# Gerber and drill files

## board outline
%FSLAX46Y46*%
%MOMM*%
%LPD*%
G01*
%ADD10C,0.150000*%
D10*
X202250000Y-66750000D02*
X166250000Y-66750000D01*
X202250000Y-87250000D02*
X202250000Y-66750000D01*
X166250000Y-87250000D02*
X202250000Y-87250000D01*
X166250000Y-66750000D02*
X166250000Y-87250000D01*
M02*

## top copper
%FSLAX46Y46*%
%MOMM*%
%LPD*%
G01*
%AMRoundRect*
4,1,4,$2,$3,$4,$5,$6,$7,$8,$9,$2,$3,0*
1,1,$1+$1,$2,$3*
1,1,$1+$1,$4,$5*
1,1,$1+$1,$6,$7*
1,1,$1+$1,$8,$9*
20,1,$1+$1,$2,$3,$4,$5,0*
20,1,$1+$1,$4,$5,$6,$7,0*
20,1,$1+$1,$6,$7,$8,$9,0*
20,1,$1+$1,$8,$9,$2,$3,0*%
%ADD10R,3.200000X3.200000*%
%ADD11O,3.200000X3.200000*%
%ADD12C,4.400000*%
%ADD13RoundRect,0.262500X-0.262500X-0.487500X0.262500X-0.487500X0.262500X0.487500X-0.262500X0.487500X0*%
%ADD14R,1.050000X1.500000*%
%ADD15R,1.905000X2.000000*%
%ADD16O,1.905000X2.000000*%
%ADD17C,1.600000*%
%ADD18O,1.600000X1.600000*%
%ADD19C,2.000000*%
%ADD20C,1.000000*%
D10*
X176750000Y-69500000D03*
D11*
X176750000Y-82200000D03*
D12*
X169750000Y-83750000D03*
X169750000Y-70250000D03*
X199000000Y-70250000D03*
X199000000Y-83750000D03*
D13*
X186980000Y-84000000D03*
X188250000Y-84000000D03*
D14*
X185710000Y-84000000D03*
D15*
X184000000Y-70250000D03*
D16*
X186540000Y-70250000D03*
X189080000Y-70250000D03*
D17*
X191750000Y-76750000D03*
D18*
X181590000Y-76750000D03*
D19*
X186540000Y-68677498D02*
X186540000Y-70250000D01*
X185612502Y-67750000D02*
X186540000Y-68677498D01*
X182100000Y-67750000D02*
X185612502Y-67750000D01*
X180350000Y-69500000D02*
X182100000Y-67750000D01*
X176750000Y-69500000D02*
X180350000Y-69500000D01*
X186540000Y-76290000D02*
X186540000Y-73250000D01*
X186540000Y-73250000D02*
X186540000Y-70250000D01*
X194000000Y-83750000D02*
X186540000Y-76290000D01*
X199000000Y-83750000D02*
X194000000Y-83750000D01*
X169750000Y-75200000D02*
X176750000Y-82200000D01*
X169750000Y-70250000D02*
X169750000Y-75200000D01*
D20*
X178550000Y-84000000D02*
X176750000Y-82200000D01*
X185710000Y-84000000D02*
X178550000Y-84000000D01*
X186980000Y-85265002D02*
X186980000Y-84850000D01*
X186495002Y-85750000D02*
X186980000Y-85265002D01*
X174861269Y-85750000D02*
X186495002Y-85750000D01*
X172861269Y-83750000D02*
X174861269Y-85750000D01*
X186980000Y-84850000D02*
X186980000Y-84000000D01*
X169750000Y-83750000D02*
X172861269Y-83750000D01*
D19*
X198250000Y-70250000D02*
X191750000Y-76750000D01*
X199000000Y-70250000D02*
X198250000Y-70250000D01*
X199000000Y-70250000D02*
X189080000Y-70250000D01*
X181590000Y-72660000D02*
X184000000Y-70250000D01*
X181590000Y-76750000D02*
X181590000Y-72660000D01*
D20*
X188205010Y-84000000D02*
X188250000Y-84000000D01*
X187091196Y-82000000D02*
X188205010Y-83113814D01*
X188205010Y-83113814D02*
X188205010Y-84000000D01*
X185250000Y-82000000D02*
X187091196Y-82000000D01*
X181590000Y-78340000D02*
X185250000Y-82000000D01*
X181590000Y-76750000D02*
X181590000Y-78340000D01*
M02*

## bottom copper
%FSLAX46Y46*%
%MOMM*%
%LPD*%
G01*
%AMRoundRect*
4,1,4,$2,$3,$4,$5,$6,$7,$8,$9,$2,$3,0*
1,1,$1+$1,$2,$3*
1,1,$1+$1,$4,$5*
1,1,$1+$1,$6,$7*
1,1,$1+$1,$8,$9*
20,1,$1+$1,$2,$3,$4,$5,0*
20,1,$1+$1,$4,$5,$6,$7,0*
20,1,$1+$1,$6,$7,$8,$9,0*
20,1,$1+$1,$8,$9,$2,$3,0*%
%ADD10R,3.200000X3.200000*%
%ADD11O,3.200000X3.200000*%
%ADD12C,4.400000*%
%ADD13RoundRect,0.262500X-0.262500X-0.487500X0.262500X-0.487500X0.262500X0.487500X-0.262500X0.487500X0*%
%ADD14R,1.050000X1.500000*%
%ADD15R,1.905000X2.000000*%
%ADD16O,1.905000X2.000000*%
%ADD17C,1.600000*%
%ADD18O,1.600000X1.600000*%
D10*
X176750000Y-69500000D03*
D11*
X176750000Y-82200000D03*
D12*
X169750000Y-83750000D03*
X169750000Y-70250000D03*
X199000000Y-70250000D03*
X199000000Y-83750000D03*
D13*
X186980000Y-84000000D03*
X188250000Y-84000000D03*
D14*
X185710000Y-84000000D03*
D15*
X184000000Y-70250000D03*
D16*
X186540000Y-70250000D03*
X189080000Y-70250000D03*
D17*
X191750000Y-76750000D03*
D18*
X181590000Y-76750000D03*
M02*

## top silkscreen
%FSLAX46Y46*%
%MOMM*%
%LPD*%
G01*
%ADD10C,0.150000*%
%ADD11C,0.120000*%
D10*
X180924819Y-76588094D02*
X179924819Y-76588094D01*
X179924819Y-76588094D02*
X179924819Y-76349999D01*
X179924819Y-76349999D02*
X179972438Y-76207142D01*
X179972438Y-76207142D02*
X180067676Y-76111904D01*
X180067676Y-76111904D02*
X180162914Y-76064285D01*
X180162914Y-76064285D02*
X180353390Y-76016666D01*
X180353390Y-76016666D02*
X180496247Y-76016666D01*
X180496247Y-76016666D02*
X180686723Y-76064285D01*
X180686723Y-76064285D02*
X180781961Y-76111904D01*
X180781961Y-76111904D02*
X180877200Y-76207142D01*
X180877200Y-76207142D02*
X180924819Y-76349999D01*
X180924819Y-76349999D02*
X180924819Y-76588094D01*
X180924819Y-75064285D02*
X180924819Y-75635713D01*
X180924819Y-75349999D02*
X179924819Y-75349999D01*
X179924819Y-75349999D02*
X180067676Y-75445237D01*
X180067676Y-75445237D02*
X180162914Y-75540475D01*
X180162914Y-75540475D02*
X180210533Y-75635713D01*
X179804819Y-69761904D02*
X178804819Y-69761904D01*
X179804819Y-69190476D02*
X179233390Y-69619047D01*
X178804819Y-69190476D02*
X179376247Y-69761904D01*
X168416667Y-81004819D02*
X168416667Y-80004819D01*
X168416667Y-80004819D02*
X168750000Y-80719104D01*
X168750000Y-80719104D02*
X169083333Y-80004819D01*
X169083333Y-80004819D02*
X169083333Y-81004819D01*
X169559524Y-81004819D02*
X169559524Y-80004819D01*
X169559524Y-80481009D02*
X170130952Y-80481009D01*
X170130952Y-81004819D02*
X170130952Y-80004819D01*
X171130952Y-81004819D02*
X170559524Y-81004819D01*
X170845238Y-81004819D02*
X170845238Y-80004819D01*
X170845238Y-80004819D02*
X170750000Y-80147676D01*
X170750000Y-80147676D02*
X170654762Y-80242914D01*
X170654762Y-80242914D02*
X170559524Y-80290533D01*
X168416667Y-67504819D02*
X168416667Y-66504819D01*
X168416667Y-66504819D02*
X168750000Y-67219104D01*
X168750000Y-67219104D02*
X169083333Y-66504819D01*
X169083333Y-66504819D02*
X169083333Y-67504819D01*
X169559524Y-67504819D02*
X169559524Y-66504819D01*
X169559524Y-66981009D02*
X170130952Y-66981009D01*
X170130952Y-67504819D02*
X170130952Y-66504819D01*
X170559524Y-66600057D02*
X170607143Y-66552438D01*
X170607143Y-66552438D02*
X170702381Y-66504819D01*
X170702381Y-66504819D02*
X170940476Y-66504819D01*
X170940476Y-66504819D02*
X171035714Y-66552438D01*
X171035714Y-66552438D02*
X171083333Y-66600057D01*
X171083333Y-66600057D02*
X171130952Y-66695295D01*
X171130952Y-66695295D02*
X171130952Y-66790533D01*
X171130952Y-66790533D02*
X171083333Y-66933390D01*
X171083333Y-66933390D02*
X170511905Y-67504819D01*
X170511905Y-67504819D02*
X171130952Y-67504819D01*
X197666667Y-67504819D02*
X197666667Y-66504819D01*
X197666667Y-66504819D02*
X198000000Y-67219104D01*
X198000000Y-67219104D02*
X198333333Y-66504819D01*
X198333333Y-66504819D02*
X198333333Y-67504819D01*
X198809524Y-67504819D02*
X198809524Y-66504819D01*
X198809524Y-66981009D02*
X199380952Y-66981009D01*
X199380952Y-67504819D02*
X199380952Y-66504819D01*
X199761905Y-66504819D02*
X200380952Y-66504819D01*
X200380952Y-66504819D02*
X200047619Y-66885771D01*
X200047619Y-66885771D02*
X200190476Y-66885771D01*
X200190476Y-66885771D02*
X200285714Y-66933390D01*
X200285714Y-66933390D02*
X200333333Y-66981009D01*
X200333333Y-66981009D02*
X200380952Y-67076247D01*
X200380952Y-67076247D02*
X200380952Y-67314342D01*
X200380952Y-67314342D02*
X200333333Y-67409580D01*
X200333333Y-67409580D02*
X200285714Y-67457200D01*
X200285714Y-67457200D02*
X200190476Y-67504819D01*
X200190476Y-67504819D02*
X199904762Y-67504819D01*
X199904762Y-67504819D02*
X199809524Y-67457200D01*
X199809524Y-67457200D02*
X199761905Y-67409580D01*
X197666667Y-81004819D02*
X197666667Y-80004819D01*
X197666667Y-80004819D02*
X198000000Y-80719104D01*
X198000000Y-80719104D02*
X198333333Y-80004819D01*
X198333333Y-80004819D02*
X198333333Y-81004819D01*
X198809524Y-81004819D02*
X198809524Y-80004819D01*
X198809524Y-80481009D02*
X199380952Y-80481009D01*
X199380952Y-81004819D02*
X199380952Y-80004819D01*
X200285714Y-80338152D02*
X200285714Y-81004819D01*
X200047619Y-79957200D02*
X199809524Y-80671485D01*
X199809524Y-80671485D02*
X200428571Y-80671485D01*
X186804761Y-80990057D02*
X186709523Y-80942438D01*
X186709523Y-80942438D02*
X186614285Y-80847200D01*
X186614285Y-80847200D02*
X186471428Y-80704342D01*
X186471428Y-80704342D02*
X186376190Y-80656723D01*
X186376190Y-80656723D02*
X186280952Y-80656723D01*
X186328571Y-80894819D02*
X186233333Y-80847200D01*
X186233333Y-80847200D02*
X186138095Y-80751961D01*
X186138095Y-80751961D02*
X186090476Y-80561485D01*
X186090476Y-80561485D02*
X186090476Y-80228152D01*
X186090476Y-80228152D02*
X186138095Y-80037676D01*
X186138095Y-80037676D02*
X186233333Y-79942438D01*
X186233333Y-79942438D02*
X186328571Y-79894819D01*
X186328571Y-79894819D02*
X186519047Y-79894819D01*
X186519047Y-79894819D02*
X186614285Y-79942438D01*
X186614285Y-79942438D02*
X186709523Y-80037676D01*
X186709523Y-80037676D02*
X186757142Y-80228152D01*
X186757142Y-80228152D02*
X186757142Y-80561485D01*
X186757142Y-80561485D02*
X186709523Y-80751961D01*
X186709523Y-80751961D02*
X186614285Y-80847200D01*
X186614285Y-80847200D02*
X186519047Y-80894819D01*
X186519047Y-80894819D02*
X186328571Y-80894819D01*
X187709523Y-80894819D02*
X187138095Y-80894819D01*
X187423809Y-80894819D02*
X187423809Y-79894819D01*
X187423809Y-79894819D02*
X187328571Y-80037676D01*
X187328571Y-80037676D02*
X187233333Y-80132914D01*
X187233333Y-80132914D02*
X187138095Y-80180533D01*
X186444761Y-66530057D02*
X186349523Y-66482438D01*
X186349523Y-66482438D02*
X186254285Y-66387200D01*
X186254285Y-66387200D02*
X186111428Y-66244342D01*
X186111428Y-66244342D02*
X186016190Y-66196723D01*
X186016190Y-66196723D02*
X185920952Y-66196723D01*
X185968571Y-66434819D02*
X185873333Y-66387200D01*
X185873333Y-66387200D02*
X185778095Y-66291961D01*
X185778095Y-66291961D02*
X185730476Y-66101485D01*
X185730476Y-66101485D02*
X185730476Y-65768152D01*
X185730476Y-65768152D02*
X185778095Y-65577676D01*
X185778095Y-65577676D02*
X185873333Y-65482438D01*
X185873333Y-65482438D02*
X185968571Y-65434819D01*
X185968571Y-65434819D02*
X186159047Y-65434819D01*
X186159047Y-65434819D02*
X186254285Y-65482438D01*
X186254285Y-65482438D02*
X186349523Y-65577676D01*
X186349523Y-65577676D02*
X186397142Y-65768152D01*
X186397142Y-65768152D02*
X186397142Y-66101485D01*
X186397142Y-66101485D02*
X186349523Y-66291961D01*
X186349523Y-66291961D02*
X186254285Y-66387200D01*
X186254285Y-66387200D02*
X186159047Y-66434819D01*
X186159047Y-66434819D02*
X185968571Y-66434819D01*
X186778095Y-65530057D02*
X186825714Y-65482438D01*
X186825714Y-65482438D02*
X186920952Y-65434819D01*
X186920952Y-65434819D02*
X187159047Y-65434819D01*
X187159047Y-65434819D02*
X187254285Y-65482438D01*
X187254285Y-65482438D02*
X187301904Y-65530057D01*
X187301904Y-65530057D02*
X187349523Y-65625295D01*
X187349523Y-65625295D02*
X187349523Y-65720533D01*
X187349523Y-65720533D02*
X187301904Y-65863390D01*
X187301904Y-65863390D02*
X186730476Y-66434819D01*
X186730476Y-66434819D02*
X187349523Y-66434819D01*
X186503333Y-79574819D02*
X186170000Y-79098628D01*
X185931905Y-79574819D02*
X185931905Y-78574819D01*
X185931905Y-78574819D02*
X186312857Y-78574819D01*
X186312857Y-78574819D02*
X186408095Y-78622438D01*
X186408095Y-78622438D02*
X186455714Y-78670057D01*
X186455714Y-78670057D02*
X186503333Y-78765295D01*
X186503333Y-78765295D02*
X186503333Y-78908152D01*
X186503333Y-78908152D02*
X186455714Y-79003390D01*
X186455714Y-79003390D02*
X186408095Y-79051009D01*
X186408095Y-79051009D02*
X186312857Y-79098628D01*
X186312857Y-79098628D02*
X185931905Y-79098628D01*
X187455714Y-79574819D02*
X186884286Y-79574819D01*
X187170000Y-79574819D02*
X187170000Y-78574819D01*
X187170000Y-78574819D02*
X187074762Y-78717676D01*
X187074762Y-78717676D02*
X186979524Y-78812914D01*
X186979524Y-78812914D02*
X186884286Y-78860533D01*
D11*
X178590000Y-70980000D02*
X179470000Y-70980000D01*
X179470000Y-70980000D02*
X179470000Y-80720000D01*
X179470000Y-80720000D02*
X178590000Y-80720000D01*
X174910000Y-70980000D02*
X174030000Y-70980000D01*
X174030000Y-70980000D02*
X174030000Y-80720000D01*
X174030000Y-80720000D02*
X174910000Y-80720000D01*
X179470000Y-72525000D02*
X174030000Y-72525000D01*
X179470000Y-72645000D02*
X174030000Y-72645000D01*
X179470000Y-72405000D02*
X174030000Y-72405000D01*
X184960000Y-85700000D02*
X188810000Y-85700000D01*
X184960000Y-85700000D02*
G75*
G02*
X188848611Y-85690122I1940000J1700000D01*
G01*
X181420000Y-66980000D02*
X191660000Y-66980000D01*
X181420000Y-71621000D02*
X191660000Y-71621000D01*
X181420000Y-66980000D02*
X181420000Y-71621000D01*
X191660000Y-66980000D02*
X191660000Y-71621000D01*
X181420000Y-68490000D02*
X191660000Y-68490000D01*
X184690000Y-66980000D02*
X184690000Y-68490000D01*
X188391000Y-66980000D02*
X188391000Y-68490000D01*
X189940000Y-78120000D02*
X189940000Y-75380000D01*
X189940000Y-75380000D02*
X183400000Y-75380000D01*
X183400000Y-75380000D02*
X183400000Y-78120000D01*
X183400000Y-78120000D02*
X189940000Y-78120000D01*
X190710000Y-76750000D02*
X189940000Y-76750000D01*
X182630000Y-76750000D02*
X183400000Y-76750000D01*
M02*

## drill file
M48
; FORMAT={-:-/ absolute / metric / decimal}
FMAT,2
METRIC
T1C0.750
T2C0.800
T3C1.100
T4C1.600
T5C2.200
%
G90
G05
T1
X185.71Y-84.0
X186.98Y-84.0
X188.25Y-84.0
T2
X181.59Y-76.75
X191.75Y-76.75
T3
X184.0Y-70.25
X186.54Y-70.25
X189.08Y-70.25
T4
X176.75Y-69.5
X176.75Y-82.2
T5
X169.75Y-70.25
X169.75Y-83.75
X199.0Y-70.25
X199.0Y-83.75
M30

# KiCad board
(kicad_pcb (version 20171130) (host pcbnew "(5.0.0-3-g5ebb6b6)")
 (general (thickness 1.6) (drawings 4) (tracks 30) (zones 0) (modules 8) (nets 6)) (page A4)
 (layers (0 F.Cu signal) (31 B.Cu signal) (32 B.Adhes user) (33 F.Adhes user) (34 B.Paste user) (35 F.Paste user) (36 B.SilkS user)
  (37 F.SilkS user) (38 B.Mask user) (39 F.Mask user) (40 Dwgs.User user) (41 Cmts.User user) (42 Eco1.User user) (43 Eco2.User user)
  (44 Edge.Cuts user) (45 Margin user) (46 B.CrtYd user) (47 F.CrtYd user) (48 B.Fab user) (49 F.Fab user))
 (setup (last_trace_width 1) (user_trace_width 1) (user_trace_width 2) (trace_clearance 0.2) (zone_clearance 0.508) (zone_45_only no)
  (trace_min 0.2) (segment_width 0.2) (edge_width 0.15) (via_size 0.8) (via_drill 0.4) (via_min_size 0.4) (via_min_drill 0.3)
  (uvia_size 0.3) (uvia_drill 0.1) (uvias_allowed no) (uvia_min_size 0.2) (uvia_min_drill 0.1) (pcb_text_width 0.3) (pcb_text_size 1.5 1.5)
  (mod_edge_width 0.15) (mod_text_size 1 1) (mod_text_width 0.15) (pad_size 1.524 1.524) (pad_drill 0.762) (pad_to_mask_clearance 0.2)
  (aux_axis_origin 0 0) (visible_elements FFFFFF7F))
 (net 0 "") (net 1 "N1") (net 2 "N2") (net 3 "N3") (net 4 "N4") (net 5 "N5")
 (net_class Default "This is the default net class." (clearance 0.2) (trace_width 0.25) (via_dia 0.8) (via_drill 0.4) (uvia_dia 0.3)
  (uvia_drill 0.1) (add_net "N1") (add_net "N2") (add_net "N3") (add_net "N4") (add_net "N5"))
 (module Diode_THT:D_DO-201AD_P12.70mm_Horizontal (layer F.Cu) (at 176.75 69.5 270)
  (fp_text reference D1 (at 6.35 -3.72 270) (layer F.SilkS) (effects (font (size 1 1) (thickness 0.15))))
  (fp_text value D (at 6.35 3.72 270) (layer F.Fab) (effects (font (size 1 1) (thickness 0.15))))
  (fp_line (start 1.48 -1.84) (end 1.48 -2.72) (layer F.SilkS) (width 0.12))
  (fp_line (start 1.48 -2.72) (end 11.22 -2.72) (layer F.SilkS) (width 0.12))
  (fp_line (start 11.22 -2.72) (end 11.22 -1.84) (layer F.SilkS) (width 0.12))
  (fp_line (start 1.48 1.84) (end 1.48 2.72) (layer F.SilkS) (width 0.12))
  (fp_line (start 1.48 2.72) (end 11.22 2.72) (layer F.SilkS) (width 0.12))
  (fp_line (start 11.22 2.72) (end 11.22 1.84) (layer F.SilkS) (width 0.12))
  (fp_line (start 3.025 -2.72) (end 3.025 2.72) (layer F.SilkS) (width 0.12))
  (fp_line (start 3.145 -2.72) (end 3.145 2.72) (layer F.SilkS) (width 0.12))
  (fp_line (start 2.905 -2.72) (end 2.905 2.72) (layer F.SilkS) (width 0.12))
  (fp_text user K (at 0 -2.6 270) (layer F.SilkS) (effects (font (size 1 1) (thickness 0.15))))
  (pad 1 thru_hole rect (at 0 0 270) (size 3.2 3.2) (drill 1.6) (layers *.Cu *.Mask) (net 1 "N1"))
  (pad 2 thru_hole oval (at 12.7 0 270) (size 3.2 3.2) (drill 1.6) (layers *.Cu *.Mask) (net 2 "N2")))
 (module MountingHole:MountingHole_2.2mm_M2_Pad (layer F.Cu) (at 169.75 83.75)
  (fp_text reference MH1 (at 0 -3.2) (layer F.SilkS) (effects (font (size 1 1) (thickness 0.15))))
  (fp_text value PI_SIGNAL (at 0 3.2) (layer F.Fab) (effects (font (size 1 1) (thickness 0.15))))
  (pad 1 thru_hole circle (at 0 0) (size 4.4 4.4) (drill 2.2) (layers *.Cu *.Mask) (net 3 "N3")))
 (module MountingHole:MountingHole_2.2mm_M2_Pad (layer F.Cu) (at 169.75 70.25)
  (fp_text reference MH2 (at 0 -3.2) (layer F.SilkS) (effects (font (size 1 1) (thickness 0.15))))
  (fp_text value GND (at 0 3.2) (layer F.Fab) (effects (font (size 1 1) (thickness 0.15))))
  (pad 1 thru_hole circle (at 0 0) (size 4.4 4.4) (drill 2.2) (layers *.Cu *.Mask) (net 2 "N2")))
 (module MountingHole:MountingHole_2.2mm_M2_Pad (layer F.Cu) (at 199 70.25)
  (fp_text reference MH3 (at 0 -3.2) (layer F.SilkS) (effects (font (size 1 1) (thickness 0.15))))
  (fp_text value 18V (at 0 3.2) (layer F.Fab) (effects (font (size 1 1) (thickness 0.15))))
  (pad 1 thru_hole circle (at 0 0) (size 4.4 4.4) (drill 2.2) (layers *.Cu *.Mask) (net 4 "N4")))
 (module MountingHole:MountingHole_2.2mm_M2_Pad (layer F.Cu) (at 199 83.75)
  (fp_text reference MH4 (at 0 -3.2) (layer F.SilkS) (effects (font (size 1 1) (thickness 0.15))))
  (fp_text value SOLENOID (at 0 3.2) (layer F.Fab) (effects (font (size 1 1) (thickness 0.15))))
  (pad 1 thru_hole circle (at 0 0) (size 4.4 4.4) (drill 2.2) (layers *.Cu *.Mask) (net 1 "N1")))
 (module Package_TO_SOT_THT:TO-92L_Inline (layer F.Cu) (at 185.71 84)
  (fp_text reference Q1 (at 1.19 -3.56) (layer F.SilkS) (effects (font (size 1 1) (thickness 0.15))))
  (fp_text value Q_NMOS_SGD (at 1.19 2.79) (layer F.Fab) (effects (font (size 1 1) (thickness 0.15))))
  (fp_line (start -0.75 1.7) (end 3.1 1.7) (layer F.SilkS) (width 0.12))
  (fp_arc (start 1.19 0) (end -0.75 1.7) (angle 262.164354) (layer F.SilkS) (width 0.12))
  (pad 2 thru_hole roundrect (at 1.27 0) (size 1.05 1.5) (drill 0.75) (layers *.Cu *.Mask) (roundrect_rratio 0.25) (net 3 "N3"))
  (pad 3 thru_hole roundrect (at 2.54 0) (size 1.05 1.5) (drill 0.75) (layers *.Cu *.Mask) (roundrect_rratio 0.25) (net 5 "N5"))
  (pad 1 thru_hole rect (at 0 0) (size 1.05 1.5) (drill 0.75) (layers *.Cu *.Mask) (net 2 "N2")))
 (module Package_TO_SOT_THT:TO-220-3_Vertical (layer F.Cu) (at 184 70.25)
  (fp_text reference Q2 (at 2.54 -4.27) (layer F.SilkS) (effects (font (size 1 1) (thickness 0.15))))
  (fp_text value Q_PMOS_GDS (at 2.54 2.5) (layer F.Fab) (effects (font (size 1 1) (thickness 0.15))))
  (fp_line (start -2.58 -3.27) (end 7.66 -3.27) (layer F.SilkS) (width 0.12))
  (fp_line (start -2.58 1.371) (end 7.66 1.371) (layer F.SilkS) (width 0.12))
  (fp_line (start -2.58 -3.27) (end -2.58 1.371) (layer F.SilkS) (width 0.12))
  (fp_line (start 7.66 -3.27) (end 7.66 1.371) (layer F.SilkS) (width 0.12))
  (fp_line (start -2.58 -1.76) (end 7.66 -1.76) (layer F.SilkS) (width 0.12))
  (fp_line (start 0.69 -3.27) (end 0.69 -1.76) (layer F.SilkS) (width 0.12))
  (fp_line (start 4.391 -3.27) (end 4.391 -1.76) (layer F.SilkS) (width 0.12))
  (pad 1 thru_hole rect (at 0 0) (size 1.905 2) (drill 1.1) (layers *.Cu *.Mask) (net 5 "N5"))
  (pad 2 thru_hole oval (at 2.54 0) (size 1.905 2) (drill 1.1) (layers *.Cu *.Mask) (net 1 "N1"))
  (pad 3 thru_hole oval (at 5.08 0) (size 1.905 2) (drill 1.1) (layers *.Cu *.Mask) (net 4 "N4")))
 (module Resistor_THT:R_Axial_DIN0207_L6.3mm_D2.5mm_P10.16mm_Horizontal (layer F.Cu) (at 191.75 76.75 180)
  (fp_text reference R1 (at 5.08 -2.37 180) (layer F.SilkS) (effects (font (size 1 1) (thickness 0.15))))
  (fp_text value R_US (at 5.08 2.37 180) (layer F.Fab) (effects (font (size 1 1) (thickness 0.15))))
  (fp_line (start 1.81 -1.37) (end 1.81 1.37) (layer F.SilkS) (width 0.12))
  (fp_line (start 1.81 1.37) (end 8.35 1.37) (layer F.SilkS) (width 0.12))
  (fp_line (start 8.35 1.37) (end 8.35 -1.37) (layer F.SilkS) (width 0.12))
  (fp_line (start 8.35 -1.37) (end 1.81 -1.37) (layer F.SilkS) (width 0.12))
  (fp_line (start 1.04 0) (end 1.81 0) (layer F.SilkS) (width 0.12))
  (fp_line (start 9.12 0) (end 8.35 0) (layer F.SilkS) (width 0.12))
  (pad 1 thru_hole circle (at 0 0 180) (size 1.6 1.6) (drill 0.8) (layers *.Cu *.Mask) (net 4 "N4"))
  (pad 2 thru_hole oval (at 10.16 0 180) (size 1.6 1.6) (drill 0.8) (layers *.Cu *.Mask) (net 5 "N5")))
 (gr_line (start 202.25 66.75) (end 166.25 66.75) (layer Edge.Cuts) (width 0.15))
 (gr_line (start 202.25 87.25) (end 202.25 66.75) (layer Edge.Cuts) (width 0.15))
 (gr_line (start 166.25 87.25) (end 202.25 87.25) (layer Edge.Cuts) (width 0.15))
 (gr_line (start 166.25 66.75) (end 166.25 87.25) (layer Edge.Cuts) (width 0.15))
 (segment (start 186.54 68.677498) (end 186.54 70.25) (width 2) (layer F.Cu) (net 1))
 (segment (start 185.612502 67.75) (end 186.54 68.677498) (width 2) (layer F.Cu) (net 1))
 (segment (start 182.1 67.75) (end 185.612502 67.75) (width 2) (layer F.Cu) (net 1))
 (segment (start 180.35 69.5) (end 182.1 67.75) (width 2) (layer F.Cu) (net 1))
 (segment (start 176.75 69.5) (end 180.35 69.5) (width 2) (layer F.Cu) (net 1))
 (segment (start 186.54 76.29) (end 186.54 73.25) (width 2) (layer F.Cu) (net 1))
 (segment (start 186.54 73.25) (end 186.54 70.25) (width 2) (layer F.Cu) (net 1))
 (segment (start 194 83.75) (end 186.54 76.29) (width 2) (layer F.Cu) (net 1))
 (segment (start 199 83.75) (end 194 83.75) (width 2) (layer F.Cu) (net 1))
 (segment (start 169.75 75.2) (end 176.75 82.2) (width 2) (layer F.Cu) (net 2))
 (segment (start 169.75 70.25) (end 169.75 75.2) (width 2) (layer F.Cu) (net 2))
 (segment (start 178.55 84) (end 176.75 82.2) (width 1) (layer F.Cu) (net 2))
 (segment (start 185.71 84) (end 178.55 84) (width 1) (layer F.Cu) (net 2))
 (segment (start 186.98 85.265002) (end 186.98 84.85) (width 1) (layer F.Cu) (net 3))
 (segment (start 186.495002 85.75) (end 186.98 85.265002) (width 1) (layer F.Cu) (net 3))
 (segment (start 174.861269 85.75) (end 186.495002 85.75) (width 1) (layer F.Cu) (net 3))
 (segment (start 172.861269 83.75) (end 174.861269 85.75) (width 1) (layer F.Cu) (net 3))
 (segment (start 186.98 84.85) (end 186.98 84) (width 1) (layer F.Cu) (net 3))
 (segment (start 169.75 83.75) (end 172.861269 83.75) (width 1) (layer F.Cu) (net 3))
 (segment (start 198.25 70.25) (end 191.75 76.75) (width 2) (layer F.Cu) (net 4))
 (segment (start 199 70.25) (end 198.25 70.25) (width 2) (layer F.Cu) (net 4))
 (segment (start 199 70.25) (end 189.08 70.25) (width 2) (layer F.Cu) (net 4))
 (segment (start 181.59 72.66) (end 184 70.25) (width 2) (layer F.Cu) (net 5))
 (segment (start 181.59 76.75) (end 181.59 72.66) (width 2) (layer F.Cu) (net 5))
 (segment (start 188.20501 84) (end 188.25 84) (width 1) (layer F.Cu) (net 5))
 (segment (start 187.091196 82) (end 188.20501 83.113814) (width 1) (layer F.Cu) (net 5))
 (segment (start 188.20501 83.113814) (end 188.20501 84) (width 1) (layer F.Cu) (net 5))
 (segment (start 185.25 82) (end 187.091196 82) (width 1) (layer F.Cu) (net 5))
 (segment (start 181.59 78.34) (end 185.25 82) (width 1) (layer F.Cu) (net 5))
 (segment (start 181.59 76.75) (end 181.59 78.34) (width 1) (layer F.Cu) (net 5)))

